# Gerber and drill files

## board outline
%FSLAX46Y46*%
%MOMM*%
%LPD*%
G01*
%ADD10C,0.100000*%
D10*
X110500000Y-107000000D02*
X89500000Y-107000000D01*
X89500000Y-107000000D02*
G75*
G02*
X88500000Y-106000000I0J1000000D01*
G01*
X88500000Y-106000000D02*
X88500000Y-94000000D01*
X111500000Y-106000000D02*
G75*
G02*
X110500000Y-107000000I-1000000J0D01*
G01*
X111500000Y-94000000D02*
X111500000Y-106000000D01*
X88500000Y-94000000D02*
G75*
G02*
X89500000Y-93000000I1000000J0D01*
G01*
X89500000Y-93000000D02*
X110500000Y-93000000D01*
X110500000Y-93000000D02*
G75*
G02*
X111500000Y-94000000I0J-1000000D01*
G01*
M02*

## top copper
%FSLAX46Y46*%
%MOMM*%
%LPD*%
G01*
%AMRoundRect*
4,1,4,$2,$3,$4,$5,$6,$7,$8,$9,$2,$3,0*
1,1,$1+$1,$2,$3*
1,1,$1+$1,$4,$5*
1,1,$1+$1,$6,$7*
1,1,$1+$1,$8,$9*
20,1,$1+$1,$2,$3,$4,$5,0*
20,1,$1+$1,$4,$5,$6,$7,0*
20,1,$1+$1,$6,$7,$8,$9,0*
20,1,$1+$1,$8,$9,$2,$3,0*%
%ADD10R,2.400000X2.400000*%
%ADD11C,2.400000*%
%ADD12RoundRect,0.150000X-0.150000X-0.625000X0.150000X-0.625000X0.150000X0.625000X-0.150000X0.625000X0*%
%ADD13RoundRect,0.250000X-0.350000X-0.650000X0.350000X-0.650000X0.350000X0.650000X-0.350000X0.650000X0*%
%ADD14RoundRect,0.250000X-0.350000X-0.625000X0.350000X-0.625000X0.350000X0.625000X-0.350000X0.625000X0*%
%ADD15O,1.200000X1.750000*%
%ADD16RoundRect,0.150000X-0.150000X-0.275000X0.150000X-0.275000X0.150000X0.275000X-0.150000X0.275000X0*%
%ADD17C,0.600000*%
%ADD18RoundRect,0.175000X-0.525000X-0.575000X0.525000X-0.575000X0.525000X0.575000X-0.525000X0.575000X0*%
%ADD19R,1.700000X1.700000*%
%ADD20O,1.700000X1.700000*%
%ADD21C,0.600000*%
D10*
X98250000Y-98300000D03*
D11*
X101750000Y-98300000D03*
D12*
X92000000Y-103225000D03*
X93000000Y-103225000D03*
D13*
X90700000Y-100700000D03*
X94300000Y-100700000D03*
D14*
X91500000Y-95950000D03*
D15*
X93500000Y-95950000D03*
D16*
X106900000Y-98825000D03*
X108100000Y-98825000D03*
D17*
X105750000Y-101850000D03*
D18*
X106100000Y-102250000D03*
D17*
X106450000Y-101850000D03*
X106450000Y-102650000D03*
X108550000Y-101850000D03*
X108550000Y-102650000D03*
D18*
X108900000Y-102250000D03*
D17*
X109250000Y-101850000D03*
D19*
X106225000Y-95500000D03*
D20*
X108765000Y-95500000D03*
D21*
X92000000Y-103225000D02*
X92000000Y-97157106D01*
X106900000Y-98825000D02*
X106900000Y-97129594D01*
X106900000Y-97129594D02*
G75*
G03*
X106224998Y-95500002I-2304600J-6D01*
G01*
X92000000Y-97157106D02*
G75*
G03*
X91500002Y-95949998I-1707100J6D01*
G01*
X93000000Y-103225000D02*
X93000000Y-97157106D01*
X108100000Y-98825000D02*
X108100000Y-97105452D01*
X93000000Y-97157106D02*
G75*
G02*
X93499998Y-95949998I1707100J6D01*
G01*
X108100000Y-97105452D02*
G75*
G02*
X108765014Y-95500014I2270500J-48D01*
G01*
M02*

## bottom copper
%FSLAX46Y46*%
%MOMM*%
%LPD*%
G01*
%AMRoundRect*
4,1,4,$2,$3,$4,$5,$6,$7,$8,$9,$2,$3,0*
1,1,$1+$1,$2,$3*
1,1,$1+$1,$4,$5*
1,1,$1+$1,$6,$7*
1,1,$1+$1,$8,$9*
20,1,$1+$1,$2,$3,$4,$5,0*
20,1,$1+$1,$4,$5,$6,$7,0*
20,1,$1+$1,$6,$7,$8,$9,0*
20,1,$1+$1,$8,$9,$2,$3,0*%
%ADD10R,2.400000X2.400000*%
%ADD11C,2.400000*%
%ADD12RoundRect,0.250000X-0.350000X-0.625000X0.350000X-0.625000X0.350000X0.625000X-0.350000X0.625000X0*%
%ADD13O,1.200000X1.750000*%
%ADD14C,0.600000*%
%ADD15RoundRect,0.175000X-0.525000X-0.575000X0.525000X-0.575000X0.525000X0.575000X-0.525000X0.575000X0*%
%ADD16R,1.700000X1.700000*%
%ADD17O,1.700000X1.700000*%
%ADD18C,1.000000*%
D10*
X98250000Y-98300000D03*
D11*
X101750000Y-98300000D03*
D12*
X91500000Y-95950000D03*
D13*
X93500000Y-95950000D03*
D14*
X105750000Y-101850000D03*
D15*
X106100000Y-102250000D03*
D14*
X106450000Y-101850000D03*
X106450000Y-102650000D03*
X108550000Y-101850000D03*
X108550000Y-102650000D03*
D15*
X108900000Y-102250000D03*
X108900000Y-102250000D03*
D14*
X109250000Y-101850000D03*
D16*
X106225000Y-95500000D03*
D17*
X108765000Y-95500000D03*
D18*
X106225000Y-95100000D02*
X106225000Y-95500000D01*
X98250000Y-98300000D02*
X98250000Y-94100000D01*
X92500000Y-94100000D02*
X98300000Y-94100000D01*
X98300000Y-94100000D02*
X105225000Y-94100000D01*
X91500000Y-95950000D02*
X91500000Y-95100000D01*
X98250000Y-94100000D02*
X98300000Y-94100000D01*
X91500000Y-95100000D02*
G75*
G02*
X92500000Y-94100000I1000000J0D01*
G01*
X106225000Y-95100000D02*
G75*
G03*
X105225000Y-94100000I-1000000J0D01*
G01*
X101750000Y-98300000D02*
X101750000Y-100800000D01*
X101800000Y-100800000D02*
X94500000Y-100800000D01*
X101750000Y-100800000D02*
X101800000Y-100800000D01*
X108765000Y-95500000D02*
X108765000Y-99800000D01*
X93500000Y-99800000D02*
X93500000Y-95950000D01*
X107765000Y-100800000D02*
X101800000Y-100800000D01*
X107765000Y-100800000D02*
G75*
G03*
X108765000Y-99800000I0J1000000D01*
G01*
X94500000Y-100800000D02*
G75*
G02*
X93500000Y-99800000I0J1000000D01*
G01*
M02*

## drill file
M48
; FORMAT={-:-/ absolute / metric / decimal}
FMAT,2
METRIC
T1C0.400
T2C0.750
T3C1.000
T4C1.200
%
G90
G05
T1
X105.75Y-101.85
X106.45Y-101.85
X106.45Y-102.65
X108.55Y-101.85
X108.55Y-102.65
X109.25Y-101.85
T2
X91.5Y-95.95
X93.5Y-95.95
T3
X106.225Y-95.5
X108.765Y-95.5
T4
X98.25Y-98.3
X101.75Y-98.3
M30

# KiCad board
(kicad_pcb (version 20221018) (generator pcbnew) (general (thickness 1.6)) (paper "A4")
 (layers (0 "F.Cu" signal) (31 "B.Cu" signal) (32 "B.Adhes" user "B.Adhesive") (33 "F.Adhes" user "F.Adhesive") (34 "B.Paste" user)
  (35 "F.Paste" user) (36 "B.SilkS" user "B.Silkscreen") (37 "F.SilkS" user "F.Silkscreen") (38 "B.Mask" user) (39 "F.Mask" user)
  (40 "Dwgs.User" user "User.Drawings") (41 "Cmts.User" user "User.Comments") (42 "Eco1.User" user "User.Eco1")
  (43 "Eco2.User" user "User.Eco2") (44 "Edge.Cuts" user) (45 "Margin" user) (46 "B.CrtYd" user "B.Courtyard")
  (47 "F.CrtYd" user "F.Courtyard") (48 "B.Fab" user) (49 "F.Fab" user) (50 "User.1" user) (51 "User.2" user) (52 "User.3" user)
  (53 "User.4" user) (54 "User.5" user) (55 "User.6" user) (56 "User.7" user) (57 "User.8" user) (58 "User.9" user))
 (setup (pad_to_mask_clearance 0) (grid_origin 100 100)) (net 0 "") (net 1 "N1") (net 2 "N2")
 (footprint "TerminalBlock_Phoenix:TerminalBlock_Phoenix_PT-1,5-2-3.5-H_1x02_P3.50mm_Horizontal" (layer "F.Cu") (at 98.25 98.3)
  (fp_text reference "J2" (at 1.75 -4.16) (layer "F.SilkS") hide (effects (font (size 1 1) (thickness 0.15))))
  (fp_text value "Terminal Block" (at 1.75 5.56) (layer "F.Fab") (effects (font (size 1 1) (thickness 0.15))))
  (pad "1" thru_hole rect (at 0 0) (size 2.4 2.4) (drill 1.2) (layers "*.Cu" "*.Mask") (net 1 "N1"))
  (pad "2" thru_hole circle (at 3.5 0) (size 2.4 2.4) (drill 1.2) (layers "*.Cu" "*.Mask") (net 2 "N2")))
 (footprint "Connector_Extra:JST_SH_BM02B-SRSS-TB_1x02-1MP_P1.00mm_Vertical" (layer "F.Cu") (at 92.5 101.9)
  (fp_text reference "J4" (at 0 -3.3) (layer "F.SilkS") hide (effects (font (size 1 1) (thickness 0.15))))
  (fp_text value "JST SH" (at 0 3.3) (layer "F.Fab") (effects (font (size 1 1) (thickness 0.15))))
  (pad "1" smd roundrect (at -0.5 1.325) (size 0.6 1.55) (layers "F.Cu" "F.Paste" "F.Mask") (roundrect_rratio 0.25) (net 1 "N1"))
  (pad "2" smd roundrect (at 0.5 1.325) (size 0.6 1.55) (layers "F.Cu" "F.Paste" "F.Mask") (roundrect_rratio 0.25) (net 2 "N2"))
  (pad "MP" smd roundrect (at -1.8 -1.2) (size 1.2 1.8) (layers "F.Cu" "F.Paste" "F.Mask") (roundrect_rratio 0.208333))
  (pad "MP" smd roundrect (at 1.8 -1.2) (size 1.2 1.8) (layers "F.Cu" "F.Paste" "F.Mask") (roundrect_rratio 0.208333)))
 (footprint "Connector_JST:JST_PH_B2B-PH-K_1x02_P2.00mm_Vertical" (layer "F.Cu") (at 91.5 95.95)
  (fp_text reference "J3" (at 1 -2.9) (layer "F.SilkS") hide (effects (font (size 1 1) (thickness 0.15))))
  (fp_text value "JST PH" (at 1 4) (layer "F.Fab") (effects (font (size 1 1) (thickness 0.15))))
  (pad "1" thru_hole roundrect (at 0 0) (size 1.2 1.75) (drill 0.75) (layers "*.Cu" "*.Mask") (roundrect_rratio 0.208333) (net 1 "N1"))
  (pad "2" thru_hole oval (at 2 0) (size 1.2 1.75) (drill 0.75) (layers "*.Cu" "*.Mask") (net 2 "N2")))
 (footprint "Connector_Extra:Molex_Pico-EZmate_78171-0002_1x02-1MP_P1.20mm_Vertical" (layer "F.Cu") (at 107.5 100.7)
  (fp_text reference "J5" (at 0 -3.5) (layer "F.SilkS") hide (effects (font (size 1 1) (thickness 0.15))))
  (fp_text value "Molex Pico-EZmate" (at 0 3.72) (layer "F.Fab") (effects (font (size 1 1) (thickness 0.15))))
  (pad "" smd roundrect (at -1.75 1.9) (size 0.7 0.8) (layers "F.Paste" "F.Mask") (roundrect_rratio 0.25))
  (pad "" smd roundrect (at 1.75 1.9) (size 0.7 0.8) (layers "F.Paste" "F.Mask") (roundrect_rratio 0.25))
  (pad "1" smd roundrect (at -0.6 -1.875) (size 0.6 0.85) (layers "F.Cu" "F.Paste" "F.Mask") (roundrect_rratio 0.25) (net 1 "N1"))
  (pad "2" smd roundrect (at 0.6 -1.875) (size 0.6 0.85) (layers "F.Cu" "F.Paste" "F.Mask") (roundrect_rratio 0.25) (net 2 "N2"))
  (pad "MP" thru_hole circle (at -1.75 1.15) (size 0.6 0.6) (drill 0.4) (layers "*.Cu"))
  (pad "MP" smd roundrect (at -1.4 1.55) (size 1.4 1.5) (layers "F.Cu") (roundrect_rratio 0.125))
  (pad "MP" smd roundrect (at -1.4 1.55) (size 1.4 1.5) (layers "B.Cu") (roundrect_rratio 0.125))
  (pad "MP" thru_hole circle (at -1.05 1.15) (size 0.6 0.6) (drill 0.4) (layers "*.Cu"))
  (pad "MP" thru_hole circle (at -1.05 1.95) (size 0.6 0.6) (drill 0.4) (layers "*.Cu"))
  (pad "MP" thru_hole circle (at 1.05 1.15) (size 0.6 0.6) (drill 0.4) (layers "*.Cu"))
  (pad "MP" thru_hole circle (at 1.05 1.95) (size 0.6 0.6) (drill 0.4) (layers "*.Cu"))
  (pad "MP" smd roundrect (at 1.4 1.55) (size 1.4 1.5) (layers "F.Cu") (roundrect_rratio 0.125))
  (pad "MP" smd roundrect (at 1.4 1.55) (size 1.4 1.5) (layers "B.Cu") (roundrect_rratio 0.125))
  (pad "MP" smd roundrect (at 1.4 1.55) (size 1.4 1.5) (layers "B.Cu") (roundrect_rratio 0.125))
  (pad "MP" thru_hole circle (at 1.75 1.15) (size 0.6 0.6) (drill 0.4) (layers "*.Cu")))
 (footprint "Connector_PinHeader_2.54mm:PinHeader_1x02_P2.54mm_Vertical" (layer "F.Cu") (at 106.225 95.5 90)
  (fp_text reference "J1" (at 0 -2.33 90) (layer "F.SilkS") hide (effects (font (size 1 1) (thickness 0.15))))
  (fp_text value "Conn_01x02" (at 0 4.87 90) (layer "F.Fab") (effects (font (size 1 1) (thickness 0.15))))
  (pad "1" thru_hole rect (at 0 0 90) (size 1.7 1.7) (drill 1) (layers "*.Cu" "*.Mask") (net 1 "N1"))
  (pad "2" thru_hole oval (at 0 2.54 90) (size 1.7 1.7) (drill 1) (layers "*.Cu" "*.Mask") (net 2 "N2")))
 (gr_line (start 110.5 107) (end 89.5 107) (stroke (width 0.1) (type default)) (layer "Edge.Cuts"))
 (gr_arc (start 89.5 107) (mid 88.792893 106.707107) (end 88.5 106) (stroke (width 0.1) (type default)) (layer "Edge.Cuts"))
 (gr_line (start 88.5 106) (end 88.5 94) (stroke (width 0.1) (type default)) (layer "Edge.Cuts"))
 (gr_arc (start 111.5 106) (mid 111.207107 106.707107) (end 110.5 107) (stroke (width 0.1) (type default)) (layer "Edge.Cuts"))
 (gr_line (start 111.5 94) (end 111.5 106) (stroke (width 0.1) (type default)) (layer "Edge.Cuts"))
 (gr_arc (start 88.5 94) (mid 88.792893 93.292893) (end 89.5 93) (stroke (width 0.1) (type default)) (layer "Edge.Cuts"))
 (gr_line (start 89.5 93) (end 110.5 93) (stroke (width 0.1) (type default)) (layer "Edge.Cuts"))
 (gr_arc (start 110.5 93) (mid 111.207107 93.292893) (end 111.5 94) (stroke (width 0.1) (type default)) (layer "Edge.Cuts"))
 (segment (start 92 103.225) (end 92 97.157106) (width 0.6) (layer "F.Cu") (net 1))
 (segment (start 106.9 98.825) (end 106.9 97.129594) (width 0.6) (layer "F.Cu") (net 1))
 (arc (start 106.9 97.129594) (mid 106.724574 96.247664) (end 106.225 95.5) (width 0.6) (layer "F.Cu") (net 1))
 (arc (start 92 97.157106) (mid 91.870054 96.503825) (end 91.5 95.95) (width 0.6) (layer "F.Cu") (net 1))
 (segment (start 106.225 95.1) (end 106.225 95.5) (width 1) (layer "B.Cu") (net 1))
 (segment (start 98.25 98.3) (end 98.25 94.1) (width 1) (layer "B.Cu") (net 1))
 (segment (start 92.5 94.1) (end 98.3 94.1) (width 1) (layer "B.Cu") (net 1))
 (segment (start 98.3 94.1) (end 105.225 94.1) (width 1) (layer "B.Cu") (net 1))
 (segment (start 91.5 95.95) (end 91.5 95.1) (width 1) (layer "B.Cu") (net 1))
 (segment (start 98.25 94.1) (end 98.3 94.1) (width 1) (layer "B.Cu") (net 1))
 (arc (start 91.5 95.1) (mid 91.792893 94.392893) (end 92.5 94.1) (width 1) (layer "B.Cu") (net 1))
 (arc (start 106.225 95.1) (mid 105.932107 94.392893) (end 105.225 94.1) (width 1) (layer "B.Cu") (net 1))
 (segment (start 93 103.225) (end 93 97.157106) (width 0.6) (layer "F.Cu") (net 2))
 (segment (start 108.1 98.825) (end 108.1 97.105452) (width 0.6) (layer "F.Cu") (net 2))
 (arc (start 93 97.157106) (mid 93.129946 96.503825) (end 93.5 95.95) (width 0.6) (layer "F.Cu") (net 2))
 (arc (start 108.1 97.105452) (mid 108.272828 96.236588) (end 108.765 95.5) (width 0.6) (layer "F.Cu") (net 2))
 (segment (start 101.75 98.3) (end 101.75 100.8) (width 1) (layer "B.Cu") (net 2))
 (segment (start 101.8 100.8) (end 94.5 100.8) (width 1) (layer "B.Cu") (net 2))
 (segment (start 101.75 100.8) (end 101.8 100.8) (width 1) (layer "B.Cu") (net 2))
 (segment (start 108.765 95.5) (end 108.765 99.8) (width 1) (layer "B.Cu") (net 2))
 (segment (start 93.5 99.8) (end 93.5 95.95) (width 1) (layer "B.Cu") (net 2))
 (segment (start 107.765 100.8) (end 101.8 100.8) (width 1) (layer "B.Cu") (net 2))
 (arc (start 107.765 100.8) (mid 108.472107 100.507107) (end 108.765 99.8) (width 1) (layer "B.Cu") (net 2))
 (arc (start 94.5 100.8) (mid 93.792893 100.507107) (end 93.5 99.8) (width 1) (layer "B.Cu") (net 2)))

